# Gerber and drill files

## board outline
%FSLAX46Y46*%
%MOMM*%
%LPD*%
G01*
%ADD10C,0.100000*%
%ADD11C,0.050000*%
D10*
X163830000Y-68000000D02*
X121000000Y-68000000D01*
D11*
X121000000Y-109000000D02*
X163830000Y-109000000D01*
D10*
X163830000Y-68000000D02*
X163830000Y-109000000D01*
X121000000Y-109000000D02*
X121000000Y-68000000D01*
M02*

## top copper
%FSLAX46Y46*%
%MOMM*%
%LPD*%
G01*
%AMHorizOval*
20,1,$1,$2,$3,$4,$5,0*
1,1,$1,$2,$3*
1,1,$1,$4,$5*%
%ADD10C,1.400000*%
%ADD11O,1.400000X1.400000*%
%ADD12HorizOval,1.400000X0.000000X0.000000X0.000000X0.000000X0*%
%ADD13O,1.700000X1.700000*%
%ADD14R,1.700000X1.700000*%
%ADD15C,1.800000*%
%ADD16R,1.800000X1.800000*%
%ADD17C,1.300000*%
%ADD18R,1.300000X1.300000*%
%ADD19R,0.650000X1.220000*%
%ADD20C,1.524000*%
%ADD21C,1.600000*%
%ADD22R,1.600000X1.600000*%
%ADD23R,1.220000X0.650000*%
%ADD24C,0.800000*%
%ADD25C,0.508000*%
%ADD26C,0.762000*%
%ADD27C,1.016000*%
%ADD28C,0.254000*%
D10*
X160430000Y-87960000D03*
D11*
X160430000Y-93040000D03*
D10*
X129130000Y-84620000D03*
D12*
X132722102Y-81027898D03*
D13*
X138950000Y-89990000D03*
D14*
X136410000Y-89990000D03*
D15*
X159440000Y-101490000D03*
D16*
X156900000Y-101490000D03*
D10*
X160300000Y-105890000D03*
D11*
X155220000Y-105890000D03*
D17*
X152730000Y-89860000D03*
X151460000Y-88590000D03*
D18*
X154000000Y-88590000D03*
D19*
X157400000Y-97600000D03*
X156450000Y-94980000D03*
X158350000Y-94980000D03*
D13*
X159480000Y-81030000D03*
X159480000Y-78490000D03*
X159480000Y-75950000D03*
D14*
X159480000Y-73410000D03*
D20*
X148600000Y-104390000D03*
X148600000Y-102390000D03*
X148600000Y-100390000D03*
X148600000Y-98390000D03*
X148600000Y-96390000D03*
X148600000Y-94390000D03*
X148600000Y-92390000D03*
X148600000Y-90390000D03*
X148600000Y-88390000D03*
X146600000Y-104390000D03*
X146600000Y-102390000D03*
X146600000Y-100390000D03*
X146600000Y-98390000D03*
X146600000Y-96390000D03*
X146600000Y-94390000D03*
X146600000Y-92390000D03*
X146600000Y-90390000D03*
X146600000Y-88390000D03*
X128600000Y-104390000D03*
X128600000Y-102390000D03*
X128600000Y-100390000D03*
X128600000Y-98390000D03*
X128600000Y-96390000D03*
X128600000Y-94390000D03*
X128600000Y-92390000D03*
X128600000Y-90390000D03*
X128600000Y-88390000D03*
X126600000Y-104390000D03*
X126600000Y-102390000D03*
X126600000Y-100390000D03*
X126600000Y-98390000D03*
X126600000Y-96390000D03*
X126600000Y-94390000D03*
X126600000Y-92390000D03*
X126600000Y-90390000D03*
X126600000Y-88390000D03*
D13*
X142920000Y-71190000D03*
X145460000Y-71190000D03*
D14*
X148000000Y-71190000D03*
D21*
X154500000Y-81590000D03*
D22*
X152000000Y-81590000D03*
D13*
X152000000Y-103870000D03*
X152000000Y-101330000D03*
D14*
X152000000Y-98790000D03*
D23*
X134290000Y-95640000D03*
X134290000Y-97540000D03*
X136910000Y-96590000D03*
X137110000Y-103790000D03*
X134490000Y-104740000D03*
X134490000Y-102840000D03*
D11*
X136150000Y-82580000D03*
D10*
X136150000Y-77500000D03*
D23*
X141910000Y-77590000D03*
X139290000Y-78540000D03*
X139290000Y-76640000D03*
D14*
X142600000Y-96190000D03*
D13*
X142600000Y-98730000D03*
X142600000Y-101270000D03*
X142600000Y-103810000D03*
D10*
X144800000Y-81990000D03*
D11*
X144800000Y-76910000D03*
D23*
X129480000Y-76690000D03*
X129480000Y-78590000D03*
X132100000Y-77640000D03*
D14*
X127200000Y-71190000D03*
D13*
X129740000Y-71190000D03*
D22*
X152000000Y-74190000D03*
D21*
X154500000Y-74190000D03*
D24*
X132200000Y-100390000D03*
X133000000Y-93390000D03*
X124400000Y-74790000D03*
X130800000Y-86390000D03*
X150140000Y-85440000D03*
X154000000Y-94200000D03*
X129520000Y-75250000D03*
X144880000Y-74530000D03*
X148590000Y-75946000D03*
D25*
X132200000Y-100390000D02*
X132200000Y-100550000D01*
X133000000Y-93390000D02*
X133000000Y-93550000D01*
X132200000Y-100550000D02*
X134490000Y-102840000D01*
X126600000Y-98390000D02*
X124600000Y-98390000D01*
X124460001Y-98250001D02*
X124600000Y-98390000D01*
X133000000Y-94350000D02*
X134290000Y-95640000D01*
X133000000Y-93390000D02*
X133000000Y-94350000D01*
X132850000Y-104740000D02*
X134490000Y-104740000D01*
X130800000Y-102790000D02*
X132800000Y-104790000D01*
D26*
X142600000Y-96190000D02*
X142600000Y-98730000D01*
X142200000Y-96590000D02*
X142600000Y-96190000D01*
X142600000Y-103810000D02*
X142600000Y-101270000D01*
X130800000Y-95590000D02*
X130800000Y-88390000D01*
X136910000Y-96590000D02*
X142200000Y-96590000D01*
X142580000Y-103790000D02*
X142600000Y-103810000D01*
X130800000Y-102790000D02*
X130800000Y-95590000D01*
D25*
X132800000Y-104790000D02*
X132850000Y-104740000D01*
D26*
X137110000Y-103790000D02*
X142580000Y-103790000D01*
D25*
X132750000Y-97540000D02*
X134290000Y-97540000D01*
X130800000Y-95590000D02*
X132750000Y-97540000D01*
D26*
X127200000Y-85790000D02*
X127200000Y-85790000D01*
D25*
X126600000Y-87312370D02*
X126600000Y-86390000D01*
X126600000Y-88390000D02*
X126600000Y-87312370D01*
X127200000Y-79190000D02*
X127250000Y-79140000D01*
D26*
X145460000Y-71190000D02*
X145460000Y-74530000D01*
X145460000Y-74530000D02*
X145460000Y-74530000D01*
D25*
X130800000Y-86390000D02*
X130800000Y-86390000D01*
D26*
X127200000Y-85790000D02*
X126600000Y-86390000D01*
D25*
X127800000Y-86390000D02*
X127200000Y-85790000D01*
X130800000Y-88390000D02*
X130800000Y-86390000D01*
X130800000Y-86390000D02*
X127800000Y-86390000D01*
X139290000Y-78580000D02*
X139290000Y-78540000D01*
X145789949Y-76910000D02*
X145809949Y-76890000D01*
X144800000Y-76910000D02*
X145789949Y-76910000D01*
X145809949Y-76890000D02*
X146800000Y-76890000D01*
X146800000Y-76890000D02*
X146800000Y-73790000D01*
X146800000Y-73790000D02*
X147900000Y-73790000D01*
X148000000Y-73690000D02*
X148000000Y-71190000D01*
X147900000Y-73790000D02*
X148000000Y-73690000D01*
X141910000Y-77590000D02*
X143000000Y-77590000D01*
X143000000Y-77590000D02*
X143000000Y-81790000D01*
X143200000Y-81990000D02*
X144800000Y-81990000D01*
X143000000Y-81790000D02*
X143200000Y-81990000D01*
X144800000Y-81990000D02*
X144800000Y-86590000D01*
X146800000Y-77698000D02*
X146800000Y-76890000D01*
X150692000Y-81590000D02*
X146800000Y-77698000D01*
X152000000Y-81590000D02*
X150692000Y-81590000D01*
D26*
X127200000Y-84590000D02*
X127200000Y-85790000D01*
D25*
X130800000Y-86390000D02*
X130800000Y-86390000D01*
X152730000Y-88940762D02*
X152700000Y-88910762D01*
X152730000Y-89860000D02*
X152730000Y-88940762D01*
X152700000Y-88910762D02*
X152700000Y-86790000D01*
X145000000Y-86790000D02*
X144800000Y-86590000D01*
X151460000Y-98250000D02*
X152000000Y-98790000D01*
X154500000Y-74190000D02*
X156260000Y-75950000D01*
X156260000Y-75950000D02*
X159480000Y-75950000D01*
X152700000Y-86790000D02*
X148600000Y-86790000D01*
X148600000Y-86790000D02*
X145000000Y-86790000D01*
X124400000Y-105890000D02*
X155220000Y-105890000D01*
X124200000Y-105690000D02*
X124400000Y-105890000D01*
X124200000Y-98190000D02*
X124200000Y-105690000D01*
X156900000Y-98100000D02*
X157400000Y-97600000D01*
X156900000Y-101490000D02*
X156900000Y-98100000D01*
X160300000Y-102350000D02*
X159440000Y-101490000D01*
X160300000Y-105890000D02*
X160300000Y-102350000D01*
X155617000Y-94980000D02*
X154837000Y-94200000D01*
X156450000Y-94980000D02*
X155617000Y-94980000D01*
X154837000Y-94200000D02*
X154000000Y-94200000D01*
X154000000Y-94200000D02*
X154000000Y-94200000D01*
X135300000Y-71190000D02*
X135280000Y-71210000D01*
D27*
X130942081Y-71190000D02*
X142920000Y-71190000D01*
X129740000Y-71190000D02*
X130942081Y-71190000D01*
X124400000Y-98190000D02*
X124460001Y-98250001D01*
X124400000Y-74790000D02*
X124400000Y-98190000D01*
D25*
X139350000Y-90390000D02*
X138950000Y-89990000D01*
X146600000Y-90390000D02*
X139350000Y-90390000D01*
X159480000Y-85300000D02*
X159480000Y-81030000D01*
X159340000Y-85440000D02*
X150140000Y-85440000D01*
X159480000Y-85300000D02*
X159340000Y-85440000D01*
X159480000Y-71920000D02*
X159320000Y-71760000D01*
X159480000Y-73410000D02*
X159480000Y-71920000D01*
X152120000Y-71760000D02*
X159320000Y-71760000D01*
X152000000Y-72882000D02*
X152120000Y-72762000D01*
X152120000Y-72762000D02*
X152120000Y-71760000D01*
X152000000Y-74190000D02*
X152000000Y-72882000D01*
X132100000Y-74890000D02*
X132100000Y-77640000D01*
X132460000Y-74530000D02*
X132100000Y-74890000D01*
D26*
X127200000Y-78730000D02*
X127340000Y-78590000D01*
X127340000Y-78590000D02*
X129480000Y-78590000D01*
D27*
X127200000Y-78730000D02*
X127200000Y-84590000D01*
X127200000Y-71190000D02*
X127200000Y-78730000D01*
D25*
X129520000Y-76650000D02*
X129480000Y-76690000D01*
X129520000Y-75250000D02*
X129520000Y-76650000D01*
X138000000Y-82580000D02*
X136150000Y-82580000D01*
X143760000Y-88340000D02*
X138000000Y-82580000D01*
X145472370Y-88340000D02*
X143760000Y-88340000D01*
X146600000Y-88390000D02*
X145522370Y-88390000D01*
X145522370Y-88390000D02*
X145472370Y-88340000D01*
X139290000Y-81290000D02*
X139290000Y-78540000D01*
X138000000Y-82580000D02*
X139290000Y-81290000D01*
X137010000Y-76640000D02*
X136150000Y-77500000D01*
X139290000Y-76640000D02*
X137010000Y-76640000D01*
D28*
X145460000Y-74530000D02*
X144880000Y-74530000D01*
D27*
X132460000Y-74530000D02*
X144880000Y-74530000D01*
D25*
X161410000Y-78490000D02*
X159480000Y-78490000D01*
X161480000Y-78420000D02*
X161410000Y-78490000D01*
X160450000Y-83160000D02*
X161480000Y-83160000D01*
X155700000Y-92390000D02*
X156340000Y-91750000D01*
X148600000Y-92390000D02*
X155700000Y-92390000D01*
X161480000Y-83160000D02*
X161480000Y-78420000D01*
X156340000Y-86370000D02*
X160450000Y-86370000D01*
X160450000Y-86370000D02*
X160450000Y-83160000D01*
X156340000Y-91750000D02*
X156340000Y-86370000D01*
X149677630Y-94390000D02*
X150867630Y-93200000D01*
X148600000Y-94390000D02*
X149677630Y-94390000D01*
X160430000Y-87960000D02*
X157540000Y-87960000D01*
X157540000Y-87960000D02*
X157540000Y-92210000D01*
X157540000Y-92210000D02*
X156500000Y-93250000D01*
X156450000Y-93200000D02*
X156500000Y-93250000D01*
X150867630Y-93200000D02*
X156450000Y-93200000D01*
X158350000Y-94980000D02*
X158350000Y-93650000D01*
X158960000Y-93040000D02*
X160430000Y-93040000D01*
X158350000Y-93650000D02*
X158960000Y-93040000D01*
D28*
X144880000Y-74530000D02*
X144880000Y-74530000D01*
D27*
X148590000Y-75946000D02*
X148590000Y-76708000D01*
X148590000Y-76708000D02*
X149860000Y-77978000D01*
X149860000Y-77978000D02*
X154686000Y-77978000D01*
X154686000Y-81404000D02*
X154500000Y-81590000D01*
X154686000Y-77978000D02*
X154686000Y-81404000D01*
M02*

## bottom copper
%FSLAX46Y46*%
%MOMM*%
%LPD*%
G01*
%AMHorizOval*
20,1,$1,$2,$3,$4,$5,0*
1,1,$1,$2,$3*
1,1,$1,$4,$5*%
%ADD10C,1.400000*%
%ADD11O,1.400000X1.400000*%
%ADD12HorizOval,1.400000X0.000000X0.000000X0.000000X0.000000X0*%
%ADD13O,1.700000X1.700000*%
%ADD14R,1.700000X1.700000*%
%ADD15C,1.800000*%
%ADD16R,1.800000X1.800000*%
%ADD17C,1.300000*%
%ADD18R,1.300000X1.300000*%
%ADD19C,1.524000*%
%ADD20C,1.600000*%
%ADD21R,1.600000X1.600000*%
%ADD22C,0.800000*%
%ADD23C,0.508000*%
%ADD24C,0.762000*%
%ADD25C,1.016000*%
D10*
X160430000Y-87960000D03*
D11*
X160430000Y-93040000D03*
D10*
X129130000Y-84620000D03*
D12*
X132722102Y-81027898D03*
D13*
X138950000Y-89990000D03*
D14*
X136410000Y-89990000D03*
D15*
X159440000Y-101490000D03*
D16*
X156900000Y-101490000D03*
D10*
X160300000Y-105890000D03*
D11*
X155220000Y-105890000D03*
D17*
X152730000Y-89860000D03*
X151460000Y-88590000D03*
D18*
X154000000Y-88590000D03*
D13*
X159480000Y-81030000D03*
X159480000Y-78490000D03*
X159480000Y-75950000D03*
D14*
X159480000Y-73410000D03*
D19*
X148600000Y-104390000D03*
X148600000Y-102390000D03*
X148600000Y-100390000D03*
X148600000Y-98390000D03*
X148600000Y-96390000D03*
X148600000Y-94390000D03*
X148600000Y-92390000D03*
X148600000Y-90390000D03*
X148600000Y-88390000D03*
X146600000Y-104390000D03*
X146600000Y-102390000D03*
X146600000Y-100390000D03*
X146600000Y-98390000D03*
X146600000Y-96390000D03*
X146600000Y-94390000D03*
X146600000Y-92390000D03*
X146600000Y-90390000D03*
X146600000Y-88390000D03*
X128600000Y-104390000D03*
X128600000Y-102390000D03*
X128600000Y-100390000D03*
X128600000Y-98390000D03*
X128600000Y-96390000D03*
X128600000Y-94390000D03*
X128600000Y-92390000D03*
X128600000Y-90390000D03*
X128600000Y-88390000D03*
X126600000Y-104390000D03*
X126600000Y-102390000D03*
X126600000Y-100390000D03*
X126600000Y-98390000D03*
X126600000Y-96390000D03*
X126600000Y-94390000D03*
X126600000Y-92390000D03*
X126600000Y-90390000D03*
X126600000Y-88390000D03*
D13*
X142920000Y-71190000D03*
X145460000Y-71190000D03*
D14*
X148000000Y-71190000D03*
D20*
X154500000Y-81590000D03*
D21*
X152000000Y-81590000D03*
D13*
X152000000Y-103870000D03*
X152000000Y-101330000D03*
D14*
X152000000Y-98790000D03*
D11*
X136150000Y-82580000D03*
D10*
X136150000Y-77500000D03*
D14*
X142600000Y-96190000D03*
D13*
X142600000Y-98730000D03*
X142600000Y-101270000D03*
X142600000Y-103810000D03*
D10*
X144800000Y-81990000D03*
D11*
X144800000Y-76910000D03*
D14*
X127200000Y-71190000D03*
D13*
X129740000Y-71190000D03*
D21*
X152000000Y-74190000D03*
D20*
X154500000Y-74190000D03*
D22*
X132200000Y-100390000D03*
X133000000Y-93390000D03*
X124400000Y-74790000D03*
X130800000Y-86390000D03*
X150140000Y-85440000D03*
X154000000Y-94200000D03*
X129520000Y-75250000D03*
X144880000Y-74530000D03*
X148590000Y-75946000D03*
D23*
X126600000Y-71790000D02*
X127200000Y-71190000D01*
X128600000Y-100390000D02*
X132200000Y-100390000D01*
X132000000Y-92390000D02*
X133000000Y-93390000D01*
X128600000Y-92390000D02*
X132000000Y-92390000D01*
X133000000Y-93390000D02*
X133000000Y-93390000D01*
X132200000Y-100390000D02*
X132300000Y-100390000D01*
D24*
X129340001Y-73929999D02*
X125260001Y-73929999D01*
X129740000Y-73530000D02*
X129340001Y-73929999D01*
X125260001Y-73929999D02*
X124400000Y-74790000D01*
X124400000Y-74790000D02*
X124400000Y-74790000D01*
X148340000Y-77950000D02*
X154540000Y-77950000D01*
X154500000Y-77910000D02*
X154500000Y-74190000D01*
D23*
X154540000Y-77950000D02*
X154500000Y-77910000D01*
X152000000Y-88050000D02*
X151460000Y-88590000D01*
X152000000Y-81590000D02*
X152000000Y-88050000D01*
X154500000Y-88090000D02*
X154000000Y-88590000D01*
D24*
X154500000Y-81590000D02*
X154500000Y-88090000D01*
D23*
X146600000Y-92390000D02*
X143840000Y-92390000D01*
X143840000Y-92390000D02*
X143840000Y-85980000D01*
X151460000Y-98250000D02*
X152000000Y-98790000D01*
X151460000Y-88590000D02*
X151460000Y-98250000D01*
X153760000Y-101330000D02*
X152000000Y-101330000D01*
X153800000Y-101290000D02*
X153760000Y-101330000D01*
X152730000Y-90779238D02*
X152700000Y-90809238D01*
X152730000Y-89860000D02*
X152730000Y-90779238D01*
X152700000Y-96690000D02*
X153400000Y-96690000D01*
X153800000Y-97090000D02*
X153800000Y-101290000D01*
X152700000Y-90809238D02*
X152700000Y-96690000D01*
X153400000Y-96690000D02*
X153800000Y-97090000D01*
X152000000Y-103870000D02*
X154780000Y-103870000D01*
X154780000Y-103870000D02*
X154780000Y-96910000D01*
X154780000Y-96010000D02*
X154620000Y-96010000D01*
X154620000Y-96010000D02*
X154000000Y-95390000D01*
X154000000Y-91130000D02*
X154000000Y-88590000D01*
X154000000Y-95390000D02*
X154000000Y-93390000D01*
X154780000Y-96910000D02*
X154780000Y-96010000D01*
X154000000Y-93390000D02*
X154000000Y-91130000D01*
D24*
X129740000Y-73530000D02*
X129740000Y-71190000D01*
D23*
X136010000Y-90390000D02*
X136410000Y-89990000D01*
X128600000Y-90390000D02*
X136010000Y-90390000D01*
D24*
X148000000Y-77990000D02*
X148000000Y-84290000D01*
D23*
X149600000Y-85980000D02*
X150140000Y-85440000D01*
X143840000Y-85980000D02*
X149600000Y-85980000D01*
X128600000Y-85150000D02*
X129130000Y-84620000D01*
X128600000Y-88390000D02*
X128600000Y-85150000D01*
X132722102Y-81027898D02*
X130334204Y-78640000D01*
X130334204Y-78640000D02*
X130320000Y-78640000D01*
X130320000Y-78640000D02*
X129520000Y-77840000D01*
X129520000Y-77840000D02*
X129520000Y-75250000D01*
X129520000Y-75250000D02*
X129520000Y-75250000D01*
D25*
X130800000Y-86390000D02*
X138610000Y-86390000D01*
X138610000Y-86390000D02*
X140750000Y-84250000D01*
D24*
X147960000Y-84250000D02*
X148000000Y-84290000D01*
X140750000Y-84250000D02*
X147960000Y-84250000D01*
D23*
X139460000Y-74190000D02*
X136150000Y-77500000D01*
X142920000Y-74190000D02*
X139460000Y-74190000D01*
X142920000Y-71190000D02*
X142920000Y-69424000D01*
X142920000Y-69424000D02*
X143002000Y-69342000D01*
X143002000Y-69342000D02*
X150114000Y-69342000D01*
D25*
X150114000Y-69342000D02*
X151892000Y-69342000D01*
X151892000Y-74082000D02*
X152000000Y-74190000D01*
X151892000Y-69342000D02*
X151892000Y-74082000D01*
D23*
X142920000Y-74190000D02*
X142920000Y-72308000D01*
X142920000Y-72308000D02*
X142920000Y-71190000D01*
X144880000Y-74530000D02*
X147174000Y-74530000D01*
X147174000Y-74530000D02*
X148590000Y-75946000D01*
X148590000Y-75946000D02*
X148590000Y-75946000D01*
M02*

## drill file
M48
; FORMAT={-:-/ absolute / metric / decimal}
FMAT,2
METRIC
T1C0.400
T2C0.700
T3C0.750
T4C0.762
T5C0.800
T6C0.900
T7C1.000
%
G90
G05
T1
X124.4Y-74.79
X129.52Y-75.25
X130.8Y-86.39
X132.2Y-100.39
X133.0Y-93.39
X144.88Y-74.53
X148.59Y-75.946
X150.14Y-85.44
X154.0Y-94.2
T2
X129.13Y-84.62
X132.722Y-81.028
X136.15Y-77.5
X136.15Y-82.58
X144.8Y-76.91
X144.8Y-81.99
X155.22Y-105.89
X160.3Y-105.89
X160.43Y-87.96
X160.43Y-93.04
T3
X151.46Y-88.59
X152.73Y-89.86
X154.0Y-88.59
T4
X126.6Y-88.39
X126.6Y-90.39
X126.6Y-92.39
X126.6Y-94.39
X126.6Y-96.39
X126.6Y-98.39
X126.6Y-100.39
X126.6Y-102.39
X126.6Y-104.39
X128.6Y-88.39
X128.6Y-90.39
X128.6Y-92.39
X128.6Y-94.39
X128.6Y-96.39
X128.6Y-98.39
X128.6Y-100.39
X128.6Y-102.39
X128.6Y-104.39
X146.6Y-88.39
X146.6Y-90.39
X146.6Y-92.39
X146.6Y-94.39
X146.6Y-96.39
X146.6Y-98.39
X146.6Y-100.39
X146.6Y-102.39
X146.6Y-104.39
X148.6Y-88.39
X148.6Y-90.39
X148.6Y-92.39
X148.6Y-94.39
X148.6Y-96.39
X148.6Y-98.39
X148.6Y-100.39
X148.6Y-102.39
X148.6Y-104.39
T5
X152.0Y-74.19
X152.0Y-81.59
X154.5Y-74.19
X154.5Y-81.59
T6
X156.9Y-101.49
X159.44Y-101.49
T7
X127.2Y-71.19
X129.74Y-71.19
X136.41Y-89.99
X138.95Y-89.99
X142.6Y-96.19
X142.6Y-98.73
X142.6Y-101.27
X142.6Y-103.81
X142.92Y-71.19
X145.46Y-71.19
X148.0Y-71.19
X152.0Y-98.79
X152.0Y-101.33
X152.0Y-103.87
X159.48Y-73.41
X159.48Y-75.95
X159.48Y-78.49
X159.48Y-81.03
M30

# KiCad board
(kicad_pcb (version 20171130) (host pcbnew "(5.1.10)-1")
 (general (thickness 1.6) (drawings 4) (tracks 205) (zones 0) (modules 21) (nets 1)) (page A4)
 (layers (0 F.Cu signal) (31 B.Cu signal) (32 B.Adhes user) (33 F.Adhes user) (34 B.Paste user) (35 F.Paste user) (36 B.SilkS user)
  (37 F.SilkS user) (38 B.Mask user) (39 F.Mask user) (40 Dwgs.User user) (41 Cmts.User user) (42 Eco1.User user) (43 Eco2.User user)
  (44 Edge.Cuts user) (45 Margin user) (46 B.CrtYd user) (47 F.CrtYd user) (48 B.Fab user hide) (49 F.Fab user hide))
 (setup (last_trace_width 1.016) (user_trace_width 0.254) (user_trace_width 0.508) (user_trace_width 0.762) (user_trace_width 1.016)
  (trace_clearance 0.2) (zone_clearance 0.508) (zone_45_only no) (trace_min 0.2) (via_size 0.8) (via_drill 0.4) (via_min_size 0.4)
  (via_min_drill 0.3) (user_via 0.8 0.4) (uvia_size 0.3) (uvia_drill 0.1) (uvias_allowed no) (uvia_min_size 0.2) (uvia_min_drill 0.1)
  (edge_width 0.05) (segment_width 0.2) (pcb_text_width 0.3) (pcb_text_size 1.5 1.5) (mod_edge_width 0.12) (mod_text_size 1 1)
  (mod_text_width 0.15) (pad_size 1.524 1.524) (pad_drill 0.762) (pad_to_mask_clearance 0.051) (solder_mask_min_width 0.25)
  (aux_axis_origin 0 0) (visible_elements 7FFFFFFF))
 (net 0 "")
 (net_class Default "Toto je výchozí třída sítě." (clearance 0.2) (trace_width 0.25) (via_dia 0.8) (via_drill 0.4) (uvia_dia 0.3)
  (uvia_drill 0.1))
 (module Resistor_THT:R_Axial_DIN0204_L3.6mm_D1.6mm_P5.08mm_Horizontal (layer F.Cu) (at 160.43 87.96 270)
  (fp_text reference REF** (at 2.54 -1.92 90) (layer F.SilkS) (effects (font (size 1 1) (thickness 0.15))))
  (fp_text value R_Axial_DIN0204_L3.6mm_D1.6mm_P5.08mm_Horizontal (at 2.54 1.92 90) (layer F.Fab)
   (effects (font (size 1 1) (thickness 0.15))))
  (pad 1 thru_hole circle (at 0 0 270) (size 1.4 1.4) (drill 0.7) (layers *.Cu *.Mask))
  (pad 2 thru_hole oval (at 5.08 0 270) (size 1.4 1.4) (drill 0.7) (layers *.Cu *.Mask)))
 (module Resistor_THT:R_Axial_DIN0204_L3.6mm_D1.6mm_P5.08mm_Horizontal (layer F.Cu) (at 129.13 84.62 45)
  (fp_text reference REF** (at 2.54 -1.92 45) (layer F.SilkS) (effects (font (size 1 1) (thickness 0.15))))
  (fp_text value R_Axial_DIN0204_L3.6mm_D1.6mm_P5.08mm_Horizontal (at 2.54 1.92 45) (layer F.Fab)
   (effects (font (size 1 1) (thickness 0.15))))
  (pad 1 thru_hole circle (at 0 0 45) (size 1.4 1.4) (drill 0.7) (layers *.Cu *.Mask))
  (pad 2 thru_hole oval (at 5.08 0 45) (size 1.4 1.4) (drill 0.7) (layers *.Cu *.Mask)))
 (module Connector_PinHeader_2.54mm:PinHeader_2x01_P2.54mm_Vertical (layer F.Cu) (at 136.41 89.99)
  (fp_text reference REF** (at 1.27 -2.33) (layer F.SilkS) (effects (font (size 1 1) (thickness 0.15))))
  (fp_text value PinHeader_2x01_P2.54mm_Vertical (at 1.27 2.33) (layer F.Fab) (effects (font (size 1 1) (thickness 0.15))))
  (pad 2 thru_hole oval (at 2.54 0) (size 1.7 1.7) (drill 1) (layers *.Cu *.Mask))
  (pad 1 thru_hole rect (at 0 0) (size 1.7 1.7) (drill 1) (layers *.Cu *.Mask)))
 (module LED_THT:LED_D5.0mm (layer F.Cu) (at 156.9 101.49)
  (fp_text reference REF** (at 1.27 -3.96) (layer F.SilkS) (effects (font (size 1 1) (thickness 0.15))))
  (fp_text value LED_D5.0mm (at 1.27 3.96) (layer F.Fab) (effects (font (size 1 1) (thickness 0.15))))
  (pad 2 thru_hole circle (at 2.54 0) (size 1.8 1.8) (drill 0.9) (layers *.Cu *.Mask))
  (pad 1 thru_hole rect (at 0 0) (size 1.8 1.8) (drill 0.9) (layers *.Cu *.Mask)))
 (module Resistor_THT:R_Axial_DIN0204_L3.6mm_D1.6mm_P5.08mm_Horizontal (layer F.Cu) (at 160.3 105.89 180)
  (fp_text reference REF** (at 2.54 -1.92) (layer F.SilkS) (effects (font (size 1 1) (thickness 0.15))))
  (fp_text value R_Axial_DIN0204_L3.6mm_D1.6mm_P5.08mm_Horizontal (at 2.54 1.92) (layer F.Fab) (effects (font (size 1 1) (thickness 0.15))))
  (pad 1 thru_hole circle (at 0 0 180) (size 1.4 1.4) (drill 0.7) (layers *.Cu *.Mask))
  (pad 2 thru_hole oval (at 5.08 0 180) (size 1.4 1.4) (drill 0.7) (layers *.Cu *.Mask)))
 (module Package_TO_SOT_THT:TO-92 (layer F.Cu) (at 154 88.59 180)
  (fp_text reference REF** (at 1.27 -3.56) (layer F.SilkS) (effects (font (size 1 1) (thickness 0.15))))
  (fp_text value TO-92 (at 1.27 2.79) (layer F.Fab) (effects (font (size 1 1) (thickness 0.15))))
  (pad 2 thru_hole circle (at 1.27 -1.27 270) (size 1.3 1.3) (drill 0.75) (layers *.Cu *.Mask))
  (pad 3 thru_hole circle (at 2.54 0 270) (size 1.3 1.3) (drill 0.75) (layers *.Cu *.Mask))
  (pad 1 thru_hole rect (at 0 0 270) (size 1.3 1.3) (drill 0.75) (layers *.Cu *.Mask)))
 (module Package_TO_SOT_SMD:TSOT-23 (layer F.Cu) (at 157.4 96.29 270)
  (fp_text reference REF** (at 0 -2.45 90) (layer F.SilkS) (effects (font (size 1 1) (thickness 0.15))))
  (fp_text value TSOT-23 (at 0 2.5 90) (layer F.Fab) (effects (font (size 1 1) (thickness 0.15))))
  (pad 3 smd rect (at 1.31 0 270) (size 1.22 0.65) (layers F.Cu F.Paste F.Mask))
  (pad 2 smd rect (at -1.31 0.95 270) (size 1.22 0.65) (layers F.Cu F.Paste F.Mask))
  (pad 1 smd rect (at -1.31 -0.95 270) (size 1.22 0.65) (layers F.Cu F.Paste F.Mask)))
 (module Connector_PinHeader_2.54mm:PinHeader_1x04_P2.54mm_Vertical (layer F.Cu) (at 159.48 73.41)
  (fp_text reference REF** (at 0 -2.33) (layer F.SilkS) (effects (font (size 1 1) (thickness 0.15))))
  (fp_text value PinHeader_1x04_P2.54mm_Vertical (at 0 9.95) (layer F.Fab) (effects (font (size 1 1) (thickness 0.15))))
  (pad 4 thru_hole oval (at 0 7.62) (size 1.7 1.7) (drill 1) (layers *.Cu *.Mask))
  (pad 3 thru_hole oval (at 0 5.08) (size 1.7 1.7) (drill 1) (layers *.Cu *.Mask))
  (pad 2 thru_hole oval (at 0 2.54) (size 1.7 1.7) (drill 1) (layers *.Cu *.Mask))
  (pad 1 thru_hole rect (at 0 0) (size 1.7 1.7) (drill 1) (layers *.Cu *.Mask)))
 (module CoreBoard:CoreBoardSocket (layer F.Cu) (at 137.6 104.39)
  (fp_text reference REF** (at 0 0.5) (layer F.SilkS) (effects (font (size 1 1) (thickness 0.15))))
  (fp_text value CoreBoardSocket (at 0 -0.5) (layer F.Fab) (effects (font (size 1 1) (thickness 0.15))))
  (pad 36 thru_hole circle (at 11 0) (size 1.524 1.524) (drill 0.762) (layers *.Cu *.Mask))
  (pad 35 thru_hole circle (at 11 -2) (size 1.524 1.524) (drill 0.762) (layers *.Cu *.Mask))
  (pad 34 thru_hole circle (at 11 -4) (size 1.524 1.524) (drill 0.762) (layers *.Cu *.Mask))
  (pad 33 thru_hole circle (at 11 -6) (size 1.524 1.524) (drill 0.762) (layers *.Cu *.Mask))
  (pad 32 thru_hole circle (at 11 -8) (size 1.524 1.524) (drill 0.762) (layers *.Cu *.Mask))
  (pad 30 thru_hole circle (at 11 -10) (size 1.524 1.524) (drill 0.762) (layers *.Cu *.Mask))
  (pad 29 thru_hole circle (at 11 -12) (size 1.524 1.524) (drill 0.762) (layers *.Cu *.Mask))
  (pad 28 thru_hole circle (at 11 -14) (size 1.524 1.524) (drill 0.762) (layers *.Cu *.Mask))
  (pad 31 thru_hole circle (at 11 -16) (size 1.524 1.524) (drill 0.762) (layers *.Cu *.Mask))
  (pad 27 thru_hole circle (at 9 0) (size 1.524 1.524) (drill 0.762) (layers *.Cu *.Mask))
  (pad 26 thru_hole circle (at 9 -2) (size 1.524 1.524) (drill 0.762) (layers *.Cu *.Mask))
  (pad 25 thru_hole circle (at 9 -4) (size 1.524 1.524) (drill 0.762) (layers *.Cu *.Mask))
  (pad 24 thru_hole circle (at 9 -6) (size 1.524 1.524) (drill 0.762) (layers *.Cu *.Mask))
  (pad 23 thru_hole circle (at 9 -8) (size 1.524 1.524) (drill 0.762) (layers *.Cu *.Mask))
  (pad 22 thru_hole circle (at 9 -10) (size 1.524 1.524) (drill 0.762) (layers *.Cu *.Mask))
  (pad 20 thru_hole circle (at 9 -12) (size 1.524 1.524) (drill 0.762) (layers *.Cu *.Mask))
  (pad 21 thru_hole circle (at 9 -14) (size 1.524 1.524) (drill 0.762) (layers *.Cu *.Mask))
  (pad 19 thru_hole circle (at 9 -16) (size 1.524 1.524) (drill 0.762) (layers *.Cu *.Mask))
  (pad 18 thru_hole circle (at -9 0) (size 1.524 1.524) (drill 0.762) (layers *.Cu *.Mask))
  (pad 17 thru_hole circle (at -9 -2) (size 1.524 1.524) (drill 0.762) (layers *.Cu *.Mask))
  (pad 16 thru_hole circle (at -9 -4) (size 1.524 1.524) (drill 0.762) (layers *.Cu *.Mask))
  (pad 15 thru_hole circle (at -9 -6) (size 1.524 1.524) (drill 0.762) (layers *.Cu *.Mask))
  (pad 14 thru_hole circle (at -9 -8) (size 1.524 1.524) (drill 0.762) (layers *.Cu *.Mask))
  (pad 13 thru_hole circle (at -9 -10) (size 1.524 1.524) (drill 0.762) (layers *.Cu *.Mask))
  (pad 12 thru_hole circle (at -9 -12) (size 1.524 1.524) (drill 0.762) (layers *.Cu *.Mask))
  (pad 11 thru_hole circle (at -9 -14) (size 1.524 1.524) (drill 0.762) (layers *.Cu *.Mask))
  (pad 10 thru_hole circle (at -9 -16) (size 1.524 1.524) (drill 0.762) (layers *.Cu *.Mask))
  (pad 9 thru_hole circle (at -11 0) (size 1.524 1.524) (drill 0.762) (layers *.Cu *.Mask))
  (pad 8 thru_hole circle (at -11 -2) (size 1.524 1.524) (drill 0.762) (layers *.Cu *.Mask))
  (pad 7 thru_hole circle (at -11 -4) (size 1.524 1.524) (drill 0.762) (layers *.Cu *.Mask))
  (pad 6 thru_hole circle (at -11 -6) (size 1.524 1.524) (drill 0.762) (layers *.Cu *.Mask))
  (pad 5 thru_hole circle (at -11 -8) (size 1.524 1.524) (drill 0.762) (layers *.Cu *.Mask))
  (pad 4 thru_hole circle (at -11 -10) (size 1.524 1.524) (drill 0.762) (layers *.Cu *.Mask))
  (pad 3 thru_hole circle (at -11 -12) (size 1.524 1.524) (drill 0.762) (layers *.Cu *.Mask))
  (pad 2 thru_hole circle (at -11 -14) (size 1.524 1.524) (drill 0.762) (layers *.Cu *.Mask))
  (pad 1 thru_hole circle (at -11 -16) (size 1.524 1.524) (drill 0.762) (layers *.Cu *.Mask)))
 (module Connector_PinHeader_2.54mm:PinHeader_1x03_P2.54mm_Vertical (layer F.Cu) (at 148 71.19 270)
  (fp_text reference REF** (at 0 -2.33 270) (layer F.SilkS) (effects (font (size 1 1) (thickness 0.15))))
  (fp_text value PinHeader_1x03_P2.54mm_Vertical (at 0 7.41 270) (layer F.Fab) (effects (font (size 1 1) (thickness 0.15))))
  (pad 3 thru_hole oval (at 0 5.08 270) (size 1.7 1.7) (drill 1) (layers *.Cu *.Mask))
  (pad 2 thru_hole oval (at 0 2.54 270) (size 1.7 1.7) (drill 1) (layers *.Cu *.Mask))
  (pad 1 thru_hole rect (at 0 0 270) (size 1.7 1.7) (drill 1) (layers *.Cu *.Mask)))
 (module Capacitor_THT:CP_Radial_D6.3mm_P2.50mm (layer F.Cu) (at 152 81.59)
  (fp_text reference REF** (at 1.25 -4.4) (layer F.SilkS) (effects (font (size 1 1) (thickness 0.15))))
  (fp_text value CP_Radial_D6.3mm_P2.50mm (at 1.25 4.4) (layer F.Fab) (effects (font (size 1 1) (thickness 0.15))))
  (pad 2 thru_hole circle (at 2.5 0) (size 1.6 1.6) (drill 0.8) (layers *.Cu *.Mask))
  (pad 1 thru_hole rect (at 0 0) (size 1.6 1.6) (drill 0.8) (layers *.Cu *.Mask)))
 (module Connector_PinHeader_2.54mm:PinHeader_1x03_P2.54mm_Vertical (layer F.Cu) (at 152 98.79)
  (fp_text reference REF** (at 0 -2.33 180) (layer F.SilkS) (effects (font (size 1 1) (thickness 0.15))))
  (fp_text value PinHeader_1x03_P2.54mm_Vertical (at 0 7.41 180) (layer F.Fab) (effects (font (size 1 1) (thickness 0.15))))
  (pad 3 thru_hole oval (at 0 5.08) (size 1.7 1.7) (drill 1) (layers *.Cu *.Mask))
  (pad 2 thru_hole oval (at 0 2.54) (size 1.7 1.7) (drill 1) (layers *.Cu *.Mask))
  (pad 1 thru_hole rect (at 0 0) (size 1.7 1.7) (drill 1) (layers *.Cu *.Mask)))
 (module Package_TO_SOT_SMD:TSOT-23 (layer F.Cu) (at 135.6 96.59)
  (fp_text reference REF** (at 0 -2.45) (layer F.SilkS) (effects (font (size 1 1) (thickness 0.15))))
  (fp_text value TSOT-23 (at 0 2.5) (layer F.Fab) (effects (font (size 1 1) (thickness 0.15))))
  (pad 1 smd rect (at -1.31 -0.95) (size 1.22 0.65) (layers F.Cu F.Paste F.Mask))
  (pad 2 smd rect (at -1.31 0.95) (size 1.22 0.65) (layers F.Cu F.Paste F.Mask))
  (pad 3 smd rect (at 1.31 0) (size 1.22 0.65) (layers F.Cu F.Paste F.Mask)))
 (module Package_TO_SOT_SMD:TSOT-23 (layer F.Cu) (at 135.8 103.79)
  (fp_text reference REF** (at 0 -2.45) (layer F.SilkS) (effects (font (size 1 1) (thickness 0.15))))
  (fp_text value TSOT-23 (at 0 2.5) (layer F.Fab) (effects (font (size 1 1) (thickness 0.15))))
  (pad 3 smd rect (at 1.31 0) (size 1.22 0.65) (layers F.Cu F.Paste F.Mask))
  (pad 2 smd rect (at -1.31 0.95) (size 1.22 0.65) (layers F.Cu F.Paste F.Mask))
  (pad 1 smd rect (at -1.31 -0.95) (size 1.22 0.65) (layers F.Cu F.Paste F.Mask)))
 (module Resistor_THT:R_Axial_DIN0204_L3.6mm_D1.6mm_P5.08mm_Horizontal (layer F.Cu) (at 136.15 77.5 270)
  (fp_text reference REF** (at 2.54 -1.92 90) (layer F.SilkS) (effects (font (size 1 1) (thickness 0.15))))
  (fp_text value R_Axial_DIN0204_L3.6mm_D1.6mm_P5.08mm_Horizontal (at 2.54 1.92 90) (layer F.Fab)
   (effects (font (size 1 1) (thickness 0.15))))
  (pad 2 thru_hole oval (at 5.08 0 270) (size 1.4 1.4) (drill 0.7) (layers *.Cu *.Mask))
  (pad 1 thru_hole circle (at 0 0 270) (size 1.4 1.4) (drill 0.7) (layers *.Cu *.Mask)))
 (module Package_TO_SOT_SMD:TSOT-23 (layer F.Cu) (at 140.6 77.59)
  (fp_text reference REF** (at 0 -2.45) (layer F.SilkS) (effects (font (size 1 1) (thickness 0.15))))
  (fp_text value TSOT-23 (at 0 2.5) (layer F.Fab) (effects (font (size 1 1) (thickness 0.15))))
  (pad 3 smd rect (at 1.31 0) (size 1.22 0.65) (layers F.Cu F.Paste F.Mask))
  (pad 2 smd rect (at -1.31 0.95) (size 1.22 0.65) (layers F.Cu F.Paste F.Mask))
  (pad 1 smd rect (at -1.31 -0.95) (size 1.22 0.65) (layers F.Cu F.Paste F.Mask)))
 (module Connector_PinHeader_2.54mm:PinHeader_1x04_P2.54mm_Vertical (layer F.Cu) (at 142.6 96.19)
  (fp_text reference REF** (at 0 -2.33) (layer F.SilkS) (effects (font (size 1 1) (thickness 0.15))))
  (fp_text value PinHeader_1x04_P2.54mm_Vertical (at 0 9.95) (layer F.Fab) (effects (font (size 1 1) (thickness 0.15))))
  (pad 1 thru_hole rect (at 0 0) (size 1.7 1.7) (drill 1) (layers *.Cu *.Mask))
  (pad 2 thru_hole oval (at 0 2.54) (size 1.7 1.7) (drill 1) (layers *.Cu *.Mask))
  (pad 3 thru_hole oval (at 0 5.08) (size 1.7 1.7) (drill 1) (layers *.Cu *.Mask))
  (pad 4 thru_hole oval (at 0 7.62) (size 1.7 1.7) (drill 1) (layers *.Cu *.Mask)))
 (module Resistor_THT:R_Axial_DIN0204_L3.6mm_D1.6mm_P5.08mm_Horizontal (layer F.Cu) (at 144.8 81.99 90)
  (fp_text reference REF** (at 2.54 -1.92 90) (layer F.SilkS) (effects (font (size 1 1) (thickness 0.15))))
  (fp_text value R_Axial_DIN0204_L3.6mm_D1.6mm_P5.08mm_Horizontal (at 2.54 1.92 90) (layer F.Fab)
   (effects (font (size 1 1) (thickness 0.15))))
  (pad 1 thru_hole circle (at 0 0 90) (size 1.4 1.4) (drill 0.7) (layers *.Cu *.Mask))
  (pad 2 thru_hole oval (at 5.08 0 90) (size 1.4 1.4) (drill 0.7) (layers *.Cu *.Mask)))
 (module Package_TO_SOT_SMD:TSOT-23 (layer F.Cu) (at 130.79 77.64)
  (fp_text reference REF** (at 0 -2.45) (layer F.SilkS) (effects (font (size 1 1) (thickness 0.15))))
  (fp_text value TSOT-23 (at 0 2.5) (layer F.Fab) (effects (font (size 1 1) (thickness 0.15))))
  (pad 1 smd rect (at -1.31 -0.95) (size 1.22 0.65) (layers F.Cu F.Paste F.Mask))
  (pad 2 smd rect (at -1.31 0.95) (size 1.22 0.65) (layers F.Cu F.Paste F.Mask))
  (pad 3 smd rect (at 1.31 0) (size 1.22 0.65) (layers F.Cu F.Paste F.Mask)))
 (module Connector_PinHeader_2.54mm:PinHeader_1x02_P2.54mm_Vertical (layer F.Cu) (at 127.2 71.19 90)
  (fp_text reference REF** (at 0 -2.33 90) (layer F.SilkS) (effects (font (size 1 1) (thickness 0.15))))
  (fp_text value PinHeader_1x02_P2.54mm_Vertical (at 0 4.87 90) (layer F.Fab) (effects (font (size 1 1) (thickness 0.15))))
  (pad 1 thru_hole rect (at 0 0 90) (size 1.7 1.7) (drill 1) (layers *.Cu *.Mask))
  (pad 2 thru_hole oval (at 0 2.54 90) (size 1.7 1.7) (drill 1) (layers *.Cu *.Mask)))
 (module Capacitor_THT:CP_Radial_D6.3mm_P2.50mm (layer F.Cu) (at 152 74.19)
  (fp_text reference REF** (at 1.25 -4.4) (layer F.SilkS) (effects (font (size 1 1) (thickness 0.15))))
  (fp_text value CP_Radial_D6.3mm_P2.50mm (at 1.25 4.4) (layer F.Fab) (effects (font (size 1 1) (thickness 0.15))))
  (pad 1 thru_hole rect (at 0 0) (size 1.6 1.6) (drill 0.8) (layers *.Cu *.Mask))
  (pad 2 thru_hole circle (at 2.5 0) (size 1.6 1.6) (drill 0.8) (layers *.Cu *.Mask)))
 (gr_line (start 163.83 68) (end 121 68) (layer Edge.Cuts) (width 0.1))
 (gr_line (start 121 109) (end 163.83 109) (layer Edge.Cuts) (width 0.05))
 (gr_line (start 163.83 68) (end 163.83 109) (layer Edge.Cuts) (width 0.1))
 (gr_line (start 121 109) (end 121 68) (layer Edge.Cuts) (width 0.1))
 (via (at 132.2 100.39) (size 0.8) (drill 0.4) (layers F.Cu B.Cu) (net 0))
 (via (at 133 93.39) (size 0.8) (drill 0.4) (layers F.Cu B.Cu) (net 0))
 (segment (start 126.6 71.79) (end 127.2 71.19) (width 0.508) (layer B.Cu) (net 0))
 (segment (start 132.2 100.39) (end 132.2 100.55) (width 0.508) (layer F.Cu) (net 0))
 (segment (start 128.6 100.39) (end 132.2 100.39) (width 0.508) (layer B.Cu) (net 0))
 (segment (start 133 93.39) (end 133 93.55) (width 0.508) (layer F.Cu) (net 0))
 (segment (start 132.2 100.55) (end 134.49 102.84) (width 0.508) (layer F.Cu) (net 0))
 (segment (start 126.6 98.39) (end 124.6 98.39) (width 0.508) (layer F.Cu) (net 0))
 (segment (start 124.460001 98.250001) (end 124.6 98.39) (width 0.508) (layer F.Cu) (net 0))
 (segment (start 132 92.39) (end 133 93.39) (width 0.508) (layer B.Cu) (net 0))
 (segment (start 128.6 92.39) (end 132 92.39) (width 0.508) (layer B.Cu) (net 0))
 (segment (start 133 93.39) (end 133 93.39) (width 0.508) (layer B.Cu) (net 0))
 (segment (start 132.2 100.39) (end 132.3 100.39) (width 0.508) (layer B.Cu) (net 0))
 (segment (start 133 94.35) (end 134.29 95.64) (width 0.508) (layer F.Cu) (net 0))
 (segment (start 133 93.39) (end 133 94.35) (width 0.508) (layer F.Cu) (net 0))
 (segment (start 132.85 104.74) (end 134.49 104.74) (width 0.508) (layer F.Cu) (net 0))
 (segment (start 130.8 102.79) (end 132.8 104.79) (width 0.508) (layer F.Cu) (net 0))
 (segment (start 142.6 96.19) (end 142.6 98.73) (width 0.762) (layer F.Cu) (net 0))
 (segment (start 142.2 96.59) (end 142.6 96.19) (width 0.762) (layer F.Cu) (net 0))
 (segment (start 142.6 103.81) (end 142.6 101.27) (width 0.762) (layer F.Cu) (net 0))
 (segment (start 130.8 95.59) (end 130.8 88.39) (width 0.762) (layer F.Cu) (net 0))
 (segment (start 136.91 96.59) (end 142.2 96.59) (width 0.762) (layer F.Cu) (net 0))
 (segment (start 142.58 103.79) (end 142.6 103.81) (width 0.762) (layer F.Cu) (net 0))
 (segment (start 130.8 102.79) (end 130.8 95.59) (width 0.762) (layer F.Cu) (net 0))
 (segment (start 132.8 104.79) (end 132.85 104.74) (width 0.508) (layer F.Cu) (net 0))
 (segment (start 137.11 103.79) (end 142.58 103.79) (width 0.762) (layer F.Cu) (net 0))
 (segment (start 132.75 97.54) (end 134.29 97.54) (width 0.508) (layer F.Cu) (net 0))
 (segment (start 130.8 95.59) (end 132.75 97.54) (width 0.508) (layer F.Cu) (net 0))
 (segment (start 127.2 85.79) (end 127.2 85.79) (width 0.762) (layer F.Cu) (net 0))
 (segment (start 126.6 87.31237) (end 126.6 86.39) (width 0.508) (layer F.Cu) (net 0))
 (segment (start 126.6 88.39) (end 126.6 87.31237) (width 0.508) (layer F.Cu) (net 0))
 (segment (start 127.2 79.19) (end 127.25 79.14) (width 0.508) (layer F.Cu) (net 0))
 (segment (start 145.46 71.19) (end 145.46 74.53) (width 0.762) (layer F.Cu) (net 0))
 (segment (start 145.46 74.53) (end 145.46 74.53) (width 0.762) (layer F.Cu) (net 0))
 (segment (start 130.8 86.39) (end 130.8 86.39) (width 0.508) (layer F.Cu) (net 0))
 (segment (start 127.2 85.79) (end 126.6 86.39) (width 0.762) (layer F.Cu) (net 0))
 (segment (start 127.8 86.39) (end 127.2 85.79) (width 0.508) (layer F.Cu) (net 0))
 (segment (start 130.8 88.39) (end 130.8 86.39) (width 0.508) (layer F.Cu) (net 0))
 (segment (start 130.8 86.39) (end 127.8 86.39) (width 0.508) (layer F.Cu) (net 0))
 (segment (start 129.340001 73.929999) (end 125.260001 73.929999) (width 0.762) (layer B.Cu) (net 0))
 (segment (start 129.74 73.53) (end 129.340001 73.929999) (width 0.762) (layer B.Cu) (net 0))
 (segment (start 125.260001 73.929999) (end 124.4 74.79) (width 0.762) (layer B.Cu) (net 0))
 (segment (start 124.4 74.79) (end 124.4 74.79) (width 0.762) (layer B.Cu) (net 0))
 (via (at 124.4 74.79) (size 0.8) (drill 0.4) (layers F.Cu B.Cu) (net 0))
 (segment (start 139.29 78.58) (end 139.29 78.54) (width 0.508) (layer F.Cu) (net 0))
 (segment (start 145.789949 76.91) (end 145.809949 76.89) (width 0.508) (layer F.Cu) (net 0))
 (segment (start 144.8 76.91) (end 145.789949 76.91) (width 0.508) (layer F.Cu) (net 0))
 (segment (start 145.809949 76.89) (end 146.8 76.89) (width 0.508) (layer F.Cu) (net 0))
 (segment (start 146.8 76.89) (end 146.8 73.79) (width 0.508) (layer F.Cu) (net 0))
 (segment (start 146.8 73.79) (end 147.9 73.79) (width 0.508) (layer F.Cu) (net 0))
 (segment (start 148 73.69) (end 148 71.19) (width 0.508) (layer F.Cu) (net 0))
 (segment (start 147.9 73.79) (end 148 73.69) (width 0.508) (layer F.Cu) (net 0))
 (segment (start 141.91 77.59) (end 143 77.59) (width 0.508) (layer F.Cu) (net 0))
 (segment (start 143 77.59) (end 143 81.79) (width 0.508) (layer F.Cu) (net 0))
 (segment (start 143.2 81.99) (end 144.8 81.99) (width 0.508) (layer F.Cu) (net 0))
 (segment (start 143 81.79) (end 143.2 81.99) (width 0.508) (layer F.Cu) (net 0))
 (segment (start 144.8 81.99) (end 144.8 86.59) (width 0.508) (layer F.Cu) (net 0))
 (segment (start 148.34 77.95) (end 154.54 77.95) (width 0.762) (layer B.Cu) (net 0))
 (segment (start 154.5 77.91) (end 154.5 74.19) (width 0.762) (layer B.Cu) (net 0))
 (segment (start 154.54 77.95) (end 154.5 77.91) (width 0.508) (layer B.Cu) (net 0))
 (segment (start 146.8 77.698) (end 146.8 76.89) (width 0.508) (layer F.Cu) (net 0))
 (segment (start 150.692 81.59) (end 146.8 77.698) (width 0.508) (layer F.Cu) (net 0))
 (segment (start 152 81.59) (end 150.692 81.59) (width 0.508) (layer F.Cu) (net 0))
 (segment (start 127.2 84.59) (end 127.2 85.79) (width 0.762) (layer F.Cu) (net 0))
 (segment (start 130.8 86.39) (end 130.8 86.39) (width 0.508) (layer F.Cu) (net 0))
 (via (at 130.8 86.39) (size 0.8) (drill 0.4) (layers F.Cu B.Cu) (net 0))
 (segment (start 152.73 88.940762) (end 152.7 88.910762) (width 0.508) (layer F.Cu) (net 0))
 (segment (start 152.73 89.86) (end 152.73 88.940762) (width 0.508) (layer F.Cu) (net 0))
 (segment (start 152.7 88.910762) (end 152.7 86.79) (width 0.508) (layer F.Cu) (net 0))
 (segment (start 145 86.79) (end 144.8 86.59) (width 0.508) (layer F.Cu) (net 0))
 (segment (start 152 88.05) (end 151.46 88.59) (width 0.508) (layer B.Cu) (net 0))
 (segment (start 152 81.59) (end 152 88.05) (width 0.508) (layer B.Cu) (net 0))
 (segment (start 154.5 88.09) (end 154 88.59) (width 0.508) (layer B.Cu) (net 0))
 (segment (start 154.5 81.59) (end 154.5 88.09) (width 0.762) (layer B.Cu) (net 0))
 (segment (start 151.46 98.25) (end 152 98.79) (width 0.508) (layer F.Cu) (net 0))
 (segment (start 154.5 74.19) (end 156.26 75.95) (width 0.508) (layer F.Cu) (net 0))
 (segment (start 156.26 75.95) (end 159.48 75.95) (width 0.508) (layer F.Cu) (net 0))
 (segment (start 146.6 92.39) (end 143.84 92.39) (width 0.508) (layer B.Cu) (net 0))
 (segment (start 143.84 92.39) (end 143.84 85.98) (width 0.508) (layer B.Cu) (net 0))
 (via (at 150.14 85.44) (size 0.8) (drill 0.4) (layers F.Cu B.Cu) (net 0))
 (segment (start 152.7 86.79) (end 148.6 86.79) (width 0.508) (layer F.Cu) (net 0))
 (segment (start 148.6 86.79) (end 145 86.79) (width 0.508) (layer F.Cu) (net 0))
 (segment (start 151.46 98.25) (end 152 98.79) (width 0.508) (layer B.Cu) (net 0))
 (segment (start 151.46 88.59) (end 151.46 98.25) (width 0.508) (layer B.Cu) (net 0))
 (segment (start 153.76 101.33) (end 152 101.33) (width 0.508) (layer B.Cu) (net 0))
 (segment (start 153.8 101.29) (end 153.76 101.33) (width 0.508) (layer B.Cu) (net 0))
 (segment (start 152.73 90.779238) (end 152.7 90.809238) (width 0.508) (layer B.Cu) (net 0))
 (segment (start 152.73 89.86) (end 152.73 90.779238) (width 0.508) (layer B.Cu) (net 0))
 (segment (start 152.7 96.69) (end 153.4 96.69) (width 0.508) (layer B.Cu) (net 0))
 (segment (start 153.8 97.09) (end 153.8 101.29) (width 0.508) (layer B.Cu) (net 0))
 (segment (start 152.7 90.809238) (end 152.7 96.69) (width 0.508) (layer B.Cu) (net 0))
 (segment (start 153.4 96.69) (end 153.8 97.09) (width 0.508) (layer B.Cu) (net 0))
 (segment (start 152 103.87) (end 154.78 103.87) (width 0.508) (layer B.Cu) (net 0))
 (segment (start 154.78 103.87) (end 154.78 96.91) (width 0.508) (layer B.Cu) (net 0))
 (segment (start 154.78 96.01) (end 154.62 96.01) (width 0.508) (layer B.Cu) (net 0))
 (segment (start 154.62 96.01) (end 154 95.39) (width 0.508) (layer B.Cu) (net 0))
 (segment (start 154 91.13) (end 154 88.59) (width 0.508) (layer B.Cu) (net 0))
 (segment (start 154 95.39) (end 154 93.39) (width 0.508) (layer B.Cu) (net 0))
 (segment (start 154.78 96.91) (end 154.78 96.01) (width 0.508) (layer B.Cu) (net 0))
 (segment (start 154 93.39) (end 154 91.13) (width 0.508) (layer B.Cu) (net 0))
 (segment (start 124.4 105.89) (end 155.22 105.89) (width 0.508) (layer F.Cu) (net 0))
 (segment (start 124.2 105.69) (end 124.4 105.89) (width 0.508) (layer F.Cu) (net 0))
 (segment (start 124.2 98.19) (end 124.2 105.69) (width 0.508) (layer F.Cu) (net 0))
 (segment (start 156.9 98.1) (end 157.4 97.6) (width 0.508) (layer F.Cu) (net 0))
 (segment (start 156.9 101.49) (end 156.9 98.1) (width 0.508) (layer F.Cu) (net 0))
 (segment (start 160.3 102.35) (end 159.44 101.49) (width 0.508) (layer F.Cu) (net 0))
 (segment (start 160.3 105.89) (end 160.3 102.35) (width 0.508) (layer F.Cu) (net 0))
 (segment (start 155.617 94.98) (end 154.837 94.2) (width 0.508) (layer F.Cu) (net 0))
 (segment (start 156.45 94.98) (end 155.617 94.98) (width 0.508) (layer F.Cu) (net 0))
 (segment (start 154.837 94.2) (end 154 94.2) (width 0.508) (layer F.Cu) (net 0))
 (segment (start 154 94.2) (end 154 94.2) (width 0.508) (layer F.Cu) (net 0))
 (via (at 154 94.2) (size 0.8) (drill 0.4) (layers F.Cu B.Cu) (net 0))
 (segment (start 129.74 73.53) (end 129.74 71.19) (width 0.762) (layer B.Cu) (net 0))
 (segment (start 135.3 71.19) (end 135.28 71.21) (width 0.508) (layer F.Cu) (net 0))
 (segment (start 130.942081 71.19) (end 142.92 71.19) (width 1.016) (layer F.Cu) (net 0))
 (segment (start 129.74 71.19) (end 130.942081 71.19) (width 1.016) (layer F.Cu) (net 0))
 (segment (start 124.4 98.19) (end 124.460001 98.250001) (width 1.016) (layer F.Cu) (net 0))
 (segment (start 124.4 74.79) (end 124.4 98.19) (width 1.016) (layer F.Cu) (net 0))
 (segment (start 136.01 90.39) (end 136.41 89.99) (width 0.508) (layer B.Cu) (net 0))
 (segment (start 128.6 90.39) (end 136.01 90.39) (width 0.508) (layer B.Cu) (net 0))
 (segment (start 139.35 90.39) (end 138.95 89.99) (width 0.508) (layer F.Cu) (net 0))
 (segment (start 146.6 90.39) (end 139.35 90.39) (width 0.508) (layer F.Cu) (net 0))
 (segment (start 148 77.99) (end 148 84.29) (width 0.762) (layer B.Cu) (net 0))
 (segment (start 149.6 85.98) (end 150.14 85.44) (width 0.508) (layer B.Cu) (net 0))
 (segment (start 143.84 85.98) (end 149.6 85.98) (width 0.508) (layer B.Cu) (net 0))
 (segment (start 159.48 85.3) (end 159.48 81.03) (width 0.508) (layer F.Cu) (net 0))
 (segment (start 159.34 85.44) (end 150.14 85.44) (width 0.508) (layer F.Cu) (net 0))
 (segment (start 159.48 85.3) (end 159.34 85.44) (width 0.508) (layer F.Cu) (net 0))
 (segment (start 159.48 71.92) (end 159.32 71.76) (width 0.508) (layer F.Cu) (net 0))
 (segment (start 159.48 73.41) (end 159.48 71.92) (width 0.508) (layer F.Cu) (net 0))
 (segment (start 152.12 71.76) (end 159.32 71.76) (width 0.508) (layer F.Cu) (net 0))
 (segment (start 152 72.882) (end 152.12 72.762) (width 0.508) (layer F.Cu) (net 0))
 (segment (start 152.12 72.762) (end 152.12 71.76) (width 0.508) (layer F.Cu) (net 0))
 (segment (start 152 74.19) (end 152 72.882) (width 0.508) (layer F.Cu) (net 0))
 (segment (start 128.6 85.15) (end 129.13 84.62) (width 0.508) (layer B.Cu) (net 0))
 (segment (start 128.6 88.39) (end 128.6 85.15) (width 0.508) (layer B.Cu) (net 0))
 (segment (start 132.722102 81.027898) (end 130.334204 78.64) (width 0.508) (layer B.Cu) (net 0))
 (segment (start 130.334204 78.64) (end 130.32 78.64) (width 0.508) (layer B.Cu) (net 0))
 (segment (start 130.32 78.64) (end 129.52 77.84) (width 0.508) (layer B.Cu) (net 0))
 (segment (start 129.52 77.84) (end 129.52 75.25) (width 0.508) (layer B.Cu) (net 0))
 (segment (start 132.1 74.89) (end 132.1 77.64) (width 0.508) (layer F.Cu) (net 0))
 (segment (start 132.46 74.53) (end 132.1 74.89) (width 0.508) (layer F.Cu) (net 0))
 (segment (start 127.2 78.73) (end 127.34 78.59) (width 0.762) (layer F.Cu) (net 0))
 (segment (start 127.34 78.59) (end 129.48 78.59) (width 0.762) (layer F.Cu) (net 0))
 (segment (start 127.2 78.73) (end 127.2 84.59) (width 1.016) (layer F.Cu) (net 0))
 (segment (start 127.2 71.19) (end 127.2 78.73) (width 1.016) (layer F.Cu) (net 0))
 (segment (start 129.52 75.25) (end 129.52 75.25) (width 0.508) (layer B.Cu) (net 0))
 (via (at 129.52 75.25) (size 0.8) (drill 0.4) (layers F.Cu B.Cu) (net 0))
 (segment (start 129.52 76.65) (end 129.48 76.69) (width 0.508) (layer F.Cu) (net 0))
 (segment (start 129.52 75.25) (end 129.52 76.65) (width 0.508) (layer F.Cu) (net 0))
 (segment (start 138 82.58) (end 136.15 82.58) (width 0.508) (layer F.Cu) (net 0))
 (segment (start 143.76 88.34) (end 138 82.58) (width 0.508) (layer F.Cu) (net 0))
 (segment (start 145.47237 88.34) (end 143.76 88.34) (width 0.508) (layer F.Cu) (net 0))
 (segment (start 146.6 88.39) (end 145.52237 88.39) (width 0.508) (layer F.Cu) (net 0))
 (segment (start 145.52237 88.39) (end 145.47237 88.34) (width 0.508) (layer F.Cu) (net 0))
 (segment (start 139.29 81.29) (end 139.29 78.54) (width 0.508) (layer F.Cu) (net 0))
 (segment (start 138 82.58) (end 139.29 81.29) (width 0.508) (layer F.Cu) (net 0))
 (segment (start 137.01 76.64) (end 136.15 77.5) (width 0.508) (layer F.Cu) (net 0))
 (segment (start 139.29 76.64) (end 137.01 76.64) (width 0.508) (layer F.Cu) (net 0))
 (segment (start 145.46 74.53) (end 144.88 74.53) (width 0.254) (layer F.Cu) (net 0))
 (segment (start 132.46 74.53) (end 144.88 74.53) (width 1.016) (layer F.Cu) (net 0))
 (segment (start 161.41 78.49) (end 159.48 78.49) (width 0.508) (layer F.Cu) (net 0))
 (segment (start 161.48 78.42) (end 161.41 78.49) (width 0.508) (layer F.Cu) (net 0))
 (segment (start 160.45 83.16) (end 161.48 83.16) (width 0.508) (layer F.Cu) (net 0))
 (segment (start 155.7 92.39) (end 156.34 91.75) (width 0.508) (layer F.Cu) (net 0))
 (segment (start 148.6 92.39) (end 155.7 92.39) (width 0.508) (layer F.Cu) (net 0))
 (segment (start 161.48 83.16) (end 161.48 78.42) (width 0.508) (layer F.Cu) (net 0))
 (segment (start 156.34 86.37) (end 160.45 86.37) (width 0.508) (layer F.Cu) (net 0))
 (segment (start 160.45 86.37) (end 160.45 83.16) (width 0.508) (layer F.Cu) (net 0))
 (segment (start 156.34 91.75) (end 156.34 86.37) (width 0.508) (layer F.Cu) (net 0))
 (segment (start 149.67763 94.39) (end 150.86763 93.2) (width 0.508) (layer F.Cu) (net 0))
 (segment (start 148.6 94.39) (end 149.67763 94.39) (width 0.508) (layer F.Cu) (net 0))
 (segment (start 160.43 87.96) (end 157.54 87.96) (width 0.508) (layer F.Cu) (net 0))
 (segment (start 157.54 87.96) (end 157.54 92.21) (width 0.508) (layer F.Cu) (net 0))
 (segment (start 157.54 92.21) (end 156.5 93.25) (width 0.508) (layer F.Cu) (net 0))
 (segment (start 156.45 93.2) (end 156.5 93.25) (width 0.508) (layer F.Cu) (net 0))
 (segment (start 150.86763 93.2) (end 156.45 93.2) (width 0.508) (layer F.Cu) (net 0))
 (segment (start 158.35 94.98) (end 158.35 93.65) (width 0.508) (layer F.Cu) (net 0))
 (segment (start 158.96 93.04) (end 160.43 93.04) (width 0.508) (layer F.Cu) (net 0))
 (segment (start 158.35 93.65) (end 158.96 93.04) (width 0.508) (layer F.Cu) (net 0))
 (segment (start 130.8 86.39) (end 138.61 86.39) (width 1.016) (layer B.Cu) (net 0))
 (segment (start 138.61 86.39) (end 140.75 84.25) (width 1.016) (layer B.Cu) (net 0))
 (segment (start 147.96 84.25) (end 148 84.29) (width 0.762) (layer B.Cu) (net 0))
 (segment (start 140.75 84.25) (end 147.96 84.25) (width 0.762) (layer B.Cu) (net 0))
 (segment (start 139.46 74.19) (end 136.15 77.5) (width 0.508) (layer B.Cu) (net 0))
 (segment (start 142.92 74.19) (end 139.46 74.19) (width 0.508) (layer B.Cu) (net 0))
 (segment (start 142.92 71.19) (end 142.92 69.424) (width 0.508) (layer B.Cu) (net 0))
 (segment (start 142.92 69.424) (end 143.002 69.342) (width 0.508) (layer B.Cu) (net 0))
 (segment (start 143.002 69.342) (end 150.114 69.342) (width 0.508) (layer B.Cu) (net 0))
 (segment (start 150.114 69.342) (end 151.892 69.342) (width 1.016) (layer B.Cu) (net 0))
 (segment (start 151.892 74.082) (end 152 74.19) (width 1.016) (layer B.Cu) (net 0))
 (segment (start 151.892 69.342) (end 151.892 74.082) (width 1.016) (layer B.Cu) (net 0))
 (segment (start 142.92 74.19) (end 142.92 72.308) (width 0.508) (layer B.Cu) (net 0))
 (segment (start 142.92 72.308) (end 142.92 71.19) (width 0.508) (layer B.Cu) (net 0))
 (segment (start 144.88 74.53) (end 144.88 74.53) (width 0.254) (layer F.Cu) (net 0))
 (via (at 144.88 74.53) (size 0.8) (drill 0.4) (layers F.Cu B.Cu) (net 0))
 (segment (start 144.88 74.53) (end 147.174 74.53) (width 0.508) (layer B.Cu) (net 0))
 (segment (start 147.174 74.53) (end 148.59 75.946) (width 0.508) (layer B.Cu) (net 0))
 (segment (start 148.59 75.946) (end 148.59 75.946) (width 0.508) (layer B.Cu) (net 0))
 (via (at 148.59 75.946) (size 0.8) (drill 0.4) (layers F.Cu B.Cu) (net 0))
 (segment (start 148.59 75.946) (end 148.59 76.708) (width 1.016) (layer F.Cu) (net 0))
 (segment (start 148.59 76.708) (end 149.86 77.978) (width 1.016) (layer F.Cu) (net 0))
 (segment (start 149.86 77.978) (end 154.686 77.978) (width 1.016) (layer F.Cu) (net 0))
 (segment (start 154.686 81.404) (end 154.5 81.59) (width 1.016) (layer F.Cu) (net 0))
 (segment (start 154.686 77.978) (end 154.686 81.404) (width 1.016) (layer F.Cu) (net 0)))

